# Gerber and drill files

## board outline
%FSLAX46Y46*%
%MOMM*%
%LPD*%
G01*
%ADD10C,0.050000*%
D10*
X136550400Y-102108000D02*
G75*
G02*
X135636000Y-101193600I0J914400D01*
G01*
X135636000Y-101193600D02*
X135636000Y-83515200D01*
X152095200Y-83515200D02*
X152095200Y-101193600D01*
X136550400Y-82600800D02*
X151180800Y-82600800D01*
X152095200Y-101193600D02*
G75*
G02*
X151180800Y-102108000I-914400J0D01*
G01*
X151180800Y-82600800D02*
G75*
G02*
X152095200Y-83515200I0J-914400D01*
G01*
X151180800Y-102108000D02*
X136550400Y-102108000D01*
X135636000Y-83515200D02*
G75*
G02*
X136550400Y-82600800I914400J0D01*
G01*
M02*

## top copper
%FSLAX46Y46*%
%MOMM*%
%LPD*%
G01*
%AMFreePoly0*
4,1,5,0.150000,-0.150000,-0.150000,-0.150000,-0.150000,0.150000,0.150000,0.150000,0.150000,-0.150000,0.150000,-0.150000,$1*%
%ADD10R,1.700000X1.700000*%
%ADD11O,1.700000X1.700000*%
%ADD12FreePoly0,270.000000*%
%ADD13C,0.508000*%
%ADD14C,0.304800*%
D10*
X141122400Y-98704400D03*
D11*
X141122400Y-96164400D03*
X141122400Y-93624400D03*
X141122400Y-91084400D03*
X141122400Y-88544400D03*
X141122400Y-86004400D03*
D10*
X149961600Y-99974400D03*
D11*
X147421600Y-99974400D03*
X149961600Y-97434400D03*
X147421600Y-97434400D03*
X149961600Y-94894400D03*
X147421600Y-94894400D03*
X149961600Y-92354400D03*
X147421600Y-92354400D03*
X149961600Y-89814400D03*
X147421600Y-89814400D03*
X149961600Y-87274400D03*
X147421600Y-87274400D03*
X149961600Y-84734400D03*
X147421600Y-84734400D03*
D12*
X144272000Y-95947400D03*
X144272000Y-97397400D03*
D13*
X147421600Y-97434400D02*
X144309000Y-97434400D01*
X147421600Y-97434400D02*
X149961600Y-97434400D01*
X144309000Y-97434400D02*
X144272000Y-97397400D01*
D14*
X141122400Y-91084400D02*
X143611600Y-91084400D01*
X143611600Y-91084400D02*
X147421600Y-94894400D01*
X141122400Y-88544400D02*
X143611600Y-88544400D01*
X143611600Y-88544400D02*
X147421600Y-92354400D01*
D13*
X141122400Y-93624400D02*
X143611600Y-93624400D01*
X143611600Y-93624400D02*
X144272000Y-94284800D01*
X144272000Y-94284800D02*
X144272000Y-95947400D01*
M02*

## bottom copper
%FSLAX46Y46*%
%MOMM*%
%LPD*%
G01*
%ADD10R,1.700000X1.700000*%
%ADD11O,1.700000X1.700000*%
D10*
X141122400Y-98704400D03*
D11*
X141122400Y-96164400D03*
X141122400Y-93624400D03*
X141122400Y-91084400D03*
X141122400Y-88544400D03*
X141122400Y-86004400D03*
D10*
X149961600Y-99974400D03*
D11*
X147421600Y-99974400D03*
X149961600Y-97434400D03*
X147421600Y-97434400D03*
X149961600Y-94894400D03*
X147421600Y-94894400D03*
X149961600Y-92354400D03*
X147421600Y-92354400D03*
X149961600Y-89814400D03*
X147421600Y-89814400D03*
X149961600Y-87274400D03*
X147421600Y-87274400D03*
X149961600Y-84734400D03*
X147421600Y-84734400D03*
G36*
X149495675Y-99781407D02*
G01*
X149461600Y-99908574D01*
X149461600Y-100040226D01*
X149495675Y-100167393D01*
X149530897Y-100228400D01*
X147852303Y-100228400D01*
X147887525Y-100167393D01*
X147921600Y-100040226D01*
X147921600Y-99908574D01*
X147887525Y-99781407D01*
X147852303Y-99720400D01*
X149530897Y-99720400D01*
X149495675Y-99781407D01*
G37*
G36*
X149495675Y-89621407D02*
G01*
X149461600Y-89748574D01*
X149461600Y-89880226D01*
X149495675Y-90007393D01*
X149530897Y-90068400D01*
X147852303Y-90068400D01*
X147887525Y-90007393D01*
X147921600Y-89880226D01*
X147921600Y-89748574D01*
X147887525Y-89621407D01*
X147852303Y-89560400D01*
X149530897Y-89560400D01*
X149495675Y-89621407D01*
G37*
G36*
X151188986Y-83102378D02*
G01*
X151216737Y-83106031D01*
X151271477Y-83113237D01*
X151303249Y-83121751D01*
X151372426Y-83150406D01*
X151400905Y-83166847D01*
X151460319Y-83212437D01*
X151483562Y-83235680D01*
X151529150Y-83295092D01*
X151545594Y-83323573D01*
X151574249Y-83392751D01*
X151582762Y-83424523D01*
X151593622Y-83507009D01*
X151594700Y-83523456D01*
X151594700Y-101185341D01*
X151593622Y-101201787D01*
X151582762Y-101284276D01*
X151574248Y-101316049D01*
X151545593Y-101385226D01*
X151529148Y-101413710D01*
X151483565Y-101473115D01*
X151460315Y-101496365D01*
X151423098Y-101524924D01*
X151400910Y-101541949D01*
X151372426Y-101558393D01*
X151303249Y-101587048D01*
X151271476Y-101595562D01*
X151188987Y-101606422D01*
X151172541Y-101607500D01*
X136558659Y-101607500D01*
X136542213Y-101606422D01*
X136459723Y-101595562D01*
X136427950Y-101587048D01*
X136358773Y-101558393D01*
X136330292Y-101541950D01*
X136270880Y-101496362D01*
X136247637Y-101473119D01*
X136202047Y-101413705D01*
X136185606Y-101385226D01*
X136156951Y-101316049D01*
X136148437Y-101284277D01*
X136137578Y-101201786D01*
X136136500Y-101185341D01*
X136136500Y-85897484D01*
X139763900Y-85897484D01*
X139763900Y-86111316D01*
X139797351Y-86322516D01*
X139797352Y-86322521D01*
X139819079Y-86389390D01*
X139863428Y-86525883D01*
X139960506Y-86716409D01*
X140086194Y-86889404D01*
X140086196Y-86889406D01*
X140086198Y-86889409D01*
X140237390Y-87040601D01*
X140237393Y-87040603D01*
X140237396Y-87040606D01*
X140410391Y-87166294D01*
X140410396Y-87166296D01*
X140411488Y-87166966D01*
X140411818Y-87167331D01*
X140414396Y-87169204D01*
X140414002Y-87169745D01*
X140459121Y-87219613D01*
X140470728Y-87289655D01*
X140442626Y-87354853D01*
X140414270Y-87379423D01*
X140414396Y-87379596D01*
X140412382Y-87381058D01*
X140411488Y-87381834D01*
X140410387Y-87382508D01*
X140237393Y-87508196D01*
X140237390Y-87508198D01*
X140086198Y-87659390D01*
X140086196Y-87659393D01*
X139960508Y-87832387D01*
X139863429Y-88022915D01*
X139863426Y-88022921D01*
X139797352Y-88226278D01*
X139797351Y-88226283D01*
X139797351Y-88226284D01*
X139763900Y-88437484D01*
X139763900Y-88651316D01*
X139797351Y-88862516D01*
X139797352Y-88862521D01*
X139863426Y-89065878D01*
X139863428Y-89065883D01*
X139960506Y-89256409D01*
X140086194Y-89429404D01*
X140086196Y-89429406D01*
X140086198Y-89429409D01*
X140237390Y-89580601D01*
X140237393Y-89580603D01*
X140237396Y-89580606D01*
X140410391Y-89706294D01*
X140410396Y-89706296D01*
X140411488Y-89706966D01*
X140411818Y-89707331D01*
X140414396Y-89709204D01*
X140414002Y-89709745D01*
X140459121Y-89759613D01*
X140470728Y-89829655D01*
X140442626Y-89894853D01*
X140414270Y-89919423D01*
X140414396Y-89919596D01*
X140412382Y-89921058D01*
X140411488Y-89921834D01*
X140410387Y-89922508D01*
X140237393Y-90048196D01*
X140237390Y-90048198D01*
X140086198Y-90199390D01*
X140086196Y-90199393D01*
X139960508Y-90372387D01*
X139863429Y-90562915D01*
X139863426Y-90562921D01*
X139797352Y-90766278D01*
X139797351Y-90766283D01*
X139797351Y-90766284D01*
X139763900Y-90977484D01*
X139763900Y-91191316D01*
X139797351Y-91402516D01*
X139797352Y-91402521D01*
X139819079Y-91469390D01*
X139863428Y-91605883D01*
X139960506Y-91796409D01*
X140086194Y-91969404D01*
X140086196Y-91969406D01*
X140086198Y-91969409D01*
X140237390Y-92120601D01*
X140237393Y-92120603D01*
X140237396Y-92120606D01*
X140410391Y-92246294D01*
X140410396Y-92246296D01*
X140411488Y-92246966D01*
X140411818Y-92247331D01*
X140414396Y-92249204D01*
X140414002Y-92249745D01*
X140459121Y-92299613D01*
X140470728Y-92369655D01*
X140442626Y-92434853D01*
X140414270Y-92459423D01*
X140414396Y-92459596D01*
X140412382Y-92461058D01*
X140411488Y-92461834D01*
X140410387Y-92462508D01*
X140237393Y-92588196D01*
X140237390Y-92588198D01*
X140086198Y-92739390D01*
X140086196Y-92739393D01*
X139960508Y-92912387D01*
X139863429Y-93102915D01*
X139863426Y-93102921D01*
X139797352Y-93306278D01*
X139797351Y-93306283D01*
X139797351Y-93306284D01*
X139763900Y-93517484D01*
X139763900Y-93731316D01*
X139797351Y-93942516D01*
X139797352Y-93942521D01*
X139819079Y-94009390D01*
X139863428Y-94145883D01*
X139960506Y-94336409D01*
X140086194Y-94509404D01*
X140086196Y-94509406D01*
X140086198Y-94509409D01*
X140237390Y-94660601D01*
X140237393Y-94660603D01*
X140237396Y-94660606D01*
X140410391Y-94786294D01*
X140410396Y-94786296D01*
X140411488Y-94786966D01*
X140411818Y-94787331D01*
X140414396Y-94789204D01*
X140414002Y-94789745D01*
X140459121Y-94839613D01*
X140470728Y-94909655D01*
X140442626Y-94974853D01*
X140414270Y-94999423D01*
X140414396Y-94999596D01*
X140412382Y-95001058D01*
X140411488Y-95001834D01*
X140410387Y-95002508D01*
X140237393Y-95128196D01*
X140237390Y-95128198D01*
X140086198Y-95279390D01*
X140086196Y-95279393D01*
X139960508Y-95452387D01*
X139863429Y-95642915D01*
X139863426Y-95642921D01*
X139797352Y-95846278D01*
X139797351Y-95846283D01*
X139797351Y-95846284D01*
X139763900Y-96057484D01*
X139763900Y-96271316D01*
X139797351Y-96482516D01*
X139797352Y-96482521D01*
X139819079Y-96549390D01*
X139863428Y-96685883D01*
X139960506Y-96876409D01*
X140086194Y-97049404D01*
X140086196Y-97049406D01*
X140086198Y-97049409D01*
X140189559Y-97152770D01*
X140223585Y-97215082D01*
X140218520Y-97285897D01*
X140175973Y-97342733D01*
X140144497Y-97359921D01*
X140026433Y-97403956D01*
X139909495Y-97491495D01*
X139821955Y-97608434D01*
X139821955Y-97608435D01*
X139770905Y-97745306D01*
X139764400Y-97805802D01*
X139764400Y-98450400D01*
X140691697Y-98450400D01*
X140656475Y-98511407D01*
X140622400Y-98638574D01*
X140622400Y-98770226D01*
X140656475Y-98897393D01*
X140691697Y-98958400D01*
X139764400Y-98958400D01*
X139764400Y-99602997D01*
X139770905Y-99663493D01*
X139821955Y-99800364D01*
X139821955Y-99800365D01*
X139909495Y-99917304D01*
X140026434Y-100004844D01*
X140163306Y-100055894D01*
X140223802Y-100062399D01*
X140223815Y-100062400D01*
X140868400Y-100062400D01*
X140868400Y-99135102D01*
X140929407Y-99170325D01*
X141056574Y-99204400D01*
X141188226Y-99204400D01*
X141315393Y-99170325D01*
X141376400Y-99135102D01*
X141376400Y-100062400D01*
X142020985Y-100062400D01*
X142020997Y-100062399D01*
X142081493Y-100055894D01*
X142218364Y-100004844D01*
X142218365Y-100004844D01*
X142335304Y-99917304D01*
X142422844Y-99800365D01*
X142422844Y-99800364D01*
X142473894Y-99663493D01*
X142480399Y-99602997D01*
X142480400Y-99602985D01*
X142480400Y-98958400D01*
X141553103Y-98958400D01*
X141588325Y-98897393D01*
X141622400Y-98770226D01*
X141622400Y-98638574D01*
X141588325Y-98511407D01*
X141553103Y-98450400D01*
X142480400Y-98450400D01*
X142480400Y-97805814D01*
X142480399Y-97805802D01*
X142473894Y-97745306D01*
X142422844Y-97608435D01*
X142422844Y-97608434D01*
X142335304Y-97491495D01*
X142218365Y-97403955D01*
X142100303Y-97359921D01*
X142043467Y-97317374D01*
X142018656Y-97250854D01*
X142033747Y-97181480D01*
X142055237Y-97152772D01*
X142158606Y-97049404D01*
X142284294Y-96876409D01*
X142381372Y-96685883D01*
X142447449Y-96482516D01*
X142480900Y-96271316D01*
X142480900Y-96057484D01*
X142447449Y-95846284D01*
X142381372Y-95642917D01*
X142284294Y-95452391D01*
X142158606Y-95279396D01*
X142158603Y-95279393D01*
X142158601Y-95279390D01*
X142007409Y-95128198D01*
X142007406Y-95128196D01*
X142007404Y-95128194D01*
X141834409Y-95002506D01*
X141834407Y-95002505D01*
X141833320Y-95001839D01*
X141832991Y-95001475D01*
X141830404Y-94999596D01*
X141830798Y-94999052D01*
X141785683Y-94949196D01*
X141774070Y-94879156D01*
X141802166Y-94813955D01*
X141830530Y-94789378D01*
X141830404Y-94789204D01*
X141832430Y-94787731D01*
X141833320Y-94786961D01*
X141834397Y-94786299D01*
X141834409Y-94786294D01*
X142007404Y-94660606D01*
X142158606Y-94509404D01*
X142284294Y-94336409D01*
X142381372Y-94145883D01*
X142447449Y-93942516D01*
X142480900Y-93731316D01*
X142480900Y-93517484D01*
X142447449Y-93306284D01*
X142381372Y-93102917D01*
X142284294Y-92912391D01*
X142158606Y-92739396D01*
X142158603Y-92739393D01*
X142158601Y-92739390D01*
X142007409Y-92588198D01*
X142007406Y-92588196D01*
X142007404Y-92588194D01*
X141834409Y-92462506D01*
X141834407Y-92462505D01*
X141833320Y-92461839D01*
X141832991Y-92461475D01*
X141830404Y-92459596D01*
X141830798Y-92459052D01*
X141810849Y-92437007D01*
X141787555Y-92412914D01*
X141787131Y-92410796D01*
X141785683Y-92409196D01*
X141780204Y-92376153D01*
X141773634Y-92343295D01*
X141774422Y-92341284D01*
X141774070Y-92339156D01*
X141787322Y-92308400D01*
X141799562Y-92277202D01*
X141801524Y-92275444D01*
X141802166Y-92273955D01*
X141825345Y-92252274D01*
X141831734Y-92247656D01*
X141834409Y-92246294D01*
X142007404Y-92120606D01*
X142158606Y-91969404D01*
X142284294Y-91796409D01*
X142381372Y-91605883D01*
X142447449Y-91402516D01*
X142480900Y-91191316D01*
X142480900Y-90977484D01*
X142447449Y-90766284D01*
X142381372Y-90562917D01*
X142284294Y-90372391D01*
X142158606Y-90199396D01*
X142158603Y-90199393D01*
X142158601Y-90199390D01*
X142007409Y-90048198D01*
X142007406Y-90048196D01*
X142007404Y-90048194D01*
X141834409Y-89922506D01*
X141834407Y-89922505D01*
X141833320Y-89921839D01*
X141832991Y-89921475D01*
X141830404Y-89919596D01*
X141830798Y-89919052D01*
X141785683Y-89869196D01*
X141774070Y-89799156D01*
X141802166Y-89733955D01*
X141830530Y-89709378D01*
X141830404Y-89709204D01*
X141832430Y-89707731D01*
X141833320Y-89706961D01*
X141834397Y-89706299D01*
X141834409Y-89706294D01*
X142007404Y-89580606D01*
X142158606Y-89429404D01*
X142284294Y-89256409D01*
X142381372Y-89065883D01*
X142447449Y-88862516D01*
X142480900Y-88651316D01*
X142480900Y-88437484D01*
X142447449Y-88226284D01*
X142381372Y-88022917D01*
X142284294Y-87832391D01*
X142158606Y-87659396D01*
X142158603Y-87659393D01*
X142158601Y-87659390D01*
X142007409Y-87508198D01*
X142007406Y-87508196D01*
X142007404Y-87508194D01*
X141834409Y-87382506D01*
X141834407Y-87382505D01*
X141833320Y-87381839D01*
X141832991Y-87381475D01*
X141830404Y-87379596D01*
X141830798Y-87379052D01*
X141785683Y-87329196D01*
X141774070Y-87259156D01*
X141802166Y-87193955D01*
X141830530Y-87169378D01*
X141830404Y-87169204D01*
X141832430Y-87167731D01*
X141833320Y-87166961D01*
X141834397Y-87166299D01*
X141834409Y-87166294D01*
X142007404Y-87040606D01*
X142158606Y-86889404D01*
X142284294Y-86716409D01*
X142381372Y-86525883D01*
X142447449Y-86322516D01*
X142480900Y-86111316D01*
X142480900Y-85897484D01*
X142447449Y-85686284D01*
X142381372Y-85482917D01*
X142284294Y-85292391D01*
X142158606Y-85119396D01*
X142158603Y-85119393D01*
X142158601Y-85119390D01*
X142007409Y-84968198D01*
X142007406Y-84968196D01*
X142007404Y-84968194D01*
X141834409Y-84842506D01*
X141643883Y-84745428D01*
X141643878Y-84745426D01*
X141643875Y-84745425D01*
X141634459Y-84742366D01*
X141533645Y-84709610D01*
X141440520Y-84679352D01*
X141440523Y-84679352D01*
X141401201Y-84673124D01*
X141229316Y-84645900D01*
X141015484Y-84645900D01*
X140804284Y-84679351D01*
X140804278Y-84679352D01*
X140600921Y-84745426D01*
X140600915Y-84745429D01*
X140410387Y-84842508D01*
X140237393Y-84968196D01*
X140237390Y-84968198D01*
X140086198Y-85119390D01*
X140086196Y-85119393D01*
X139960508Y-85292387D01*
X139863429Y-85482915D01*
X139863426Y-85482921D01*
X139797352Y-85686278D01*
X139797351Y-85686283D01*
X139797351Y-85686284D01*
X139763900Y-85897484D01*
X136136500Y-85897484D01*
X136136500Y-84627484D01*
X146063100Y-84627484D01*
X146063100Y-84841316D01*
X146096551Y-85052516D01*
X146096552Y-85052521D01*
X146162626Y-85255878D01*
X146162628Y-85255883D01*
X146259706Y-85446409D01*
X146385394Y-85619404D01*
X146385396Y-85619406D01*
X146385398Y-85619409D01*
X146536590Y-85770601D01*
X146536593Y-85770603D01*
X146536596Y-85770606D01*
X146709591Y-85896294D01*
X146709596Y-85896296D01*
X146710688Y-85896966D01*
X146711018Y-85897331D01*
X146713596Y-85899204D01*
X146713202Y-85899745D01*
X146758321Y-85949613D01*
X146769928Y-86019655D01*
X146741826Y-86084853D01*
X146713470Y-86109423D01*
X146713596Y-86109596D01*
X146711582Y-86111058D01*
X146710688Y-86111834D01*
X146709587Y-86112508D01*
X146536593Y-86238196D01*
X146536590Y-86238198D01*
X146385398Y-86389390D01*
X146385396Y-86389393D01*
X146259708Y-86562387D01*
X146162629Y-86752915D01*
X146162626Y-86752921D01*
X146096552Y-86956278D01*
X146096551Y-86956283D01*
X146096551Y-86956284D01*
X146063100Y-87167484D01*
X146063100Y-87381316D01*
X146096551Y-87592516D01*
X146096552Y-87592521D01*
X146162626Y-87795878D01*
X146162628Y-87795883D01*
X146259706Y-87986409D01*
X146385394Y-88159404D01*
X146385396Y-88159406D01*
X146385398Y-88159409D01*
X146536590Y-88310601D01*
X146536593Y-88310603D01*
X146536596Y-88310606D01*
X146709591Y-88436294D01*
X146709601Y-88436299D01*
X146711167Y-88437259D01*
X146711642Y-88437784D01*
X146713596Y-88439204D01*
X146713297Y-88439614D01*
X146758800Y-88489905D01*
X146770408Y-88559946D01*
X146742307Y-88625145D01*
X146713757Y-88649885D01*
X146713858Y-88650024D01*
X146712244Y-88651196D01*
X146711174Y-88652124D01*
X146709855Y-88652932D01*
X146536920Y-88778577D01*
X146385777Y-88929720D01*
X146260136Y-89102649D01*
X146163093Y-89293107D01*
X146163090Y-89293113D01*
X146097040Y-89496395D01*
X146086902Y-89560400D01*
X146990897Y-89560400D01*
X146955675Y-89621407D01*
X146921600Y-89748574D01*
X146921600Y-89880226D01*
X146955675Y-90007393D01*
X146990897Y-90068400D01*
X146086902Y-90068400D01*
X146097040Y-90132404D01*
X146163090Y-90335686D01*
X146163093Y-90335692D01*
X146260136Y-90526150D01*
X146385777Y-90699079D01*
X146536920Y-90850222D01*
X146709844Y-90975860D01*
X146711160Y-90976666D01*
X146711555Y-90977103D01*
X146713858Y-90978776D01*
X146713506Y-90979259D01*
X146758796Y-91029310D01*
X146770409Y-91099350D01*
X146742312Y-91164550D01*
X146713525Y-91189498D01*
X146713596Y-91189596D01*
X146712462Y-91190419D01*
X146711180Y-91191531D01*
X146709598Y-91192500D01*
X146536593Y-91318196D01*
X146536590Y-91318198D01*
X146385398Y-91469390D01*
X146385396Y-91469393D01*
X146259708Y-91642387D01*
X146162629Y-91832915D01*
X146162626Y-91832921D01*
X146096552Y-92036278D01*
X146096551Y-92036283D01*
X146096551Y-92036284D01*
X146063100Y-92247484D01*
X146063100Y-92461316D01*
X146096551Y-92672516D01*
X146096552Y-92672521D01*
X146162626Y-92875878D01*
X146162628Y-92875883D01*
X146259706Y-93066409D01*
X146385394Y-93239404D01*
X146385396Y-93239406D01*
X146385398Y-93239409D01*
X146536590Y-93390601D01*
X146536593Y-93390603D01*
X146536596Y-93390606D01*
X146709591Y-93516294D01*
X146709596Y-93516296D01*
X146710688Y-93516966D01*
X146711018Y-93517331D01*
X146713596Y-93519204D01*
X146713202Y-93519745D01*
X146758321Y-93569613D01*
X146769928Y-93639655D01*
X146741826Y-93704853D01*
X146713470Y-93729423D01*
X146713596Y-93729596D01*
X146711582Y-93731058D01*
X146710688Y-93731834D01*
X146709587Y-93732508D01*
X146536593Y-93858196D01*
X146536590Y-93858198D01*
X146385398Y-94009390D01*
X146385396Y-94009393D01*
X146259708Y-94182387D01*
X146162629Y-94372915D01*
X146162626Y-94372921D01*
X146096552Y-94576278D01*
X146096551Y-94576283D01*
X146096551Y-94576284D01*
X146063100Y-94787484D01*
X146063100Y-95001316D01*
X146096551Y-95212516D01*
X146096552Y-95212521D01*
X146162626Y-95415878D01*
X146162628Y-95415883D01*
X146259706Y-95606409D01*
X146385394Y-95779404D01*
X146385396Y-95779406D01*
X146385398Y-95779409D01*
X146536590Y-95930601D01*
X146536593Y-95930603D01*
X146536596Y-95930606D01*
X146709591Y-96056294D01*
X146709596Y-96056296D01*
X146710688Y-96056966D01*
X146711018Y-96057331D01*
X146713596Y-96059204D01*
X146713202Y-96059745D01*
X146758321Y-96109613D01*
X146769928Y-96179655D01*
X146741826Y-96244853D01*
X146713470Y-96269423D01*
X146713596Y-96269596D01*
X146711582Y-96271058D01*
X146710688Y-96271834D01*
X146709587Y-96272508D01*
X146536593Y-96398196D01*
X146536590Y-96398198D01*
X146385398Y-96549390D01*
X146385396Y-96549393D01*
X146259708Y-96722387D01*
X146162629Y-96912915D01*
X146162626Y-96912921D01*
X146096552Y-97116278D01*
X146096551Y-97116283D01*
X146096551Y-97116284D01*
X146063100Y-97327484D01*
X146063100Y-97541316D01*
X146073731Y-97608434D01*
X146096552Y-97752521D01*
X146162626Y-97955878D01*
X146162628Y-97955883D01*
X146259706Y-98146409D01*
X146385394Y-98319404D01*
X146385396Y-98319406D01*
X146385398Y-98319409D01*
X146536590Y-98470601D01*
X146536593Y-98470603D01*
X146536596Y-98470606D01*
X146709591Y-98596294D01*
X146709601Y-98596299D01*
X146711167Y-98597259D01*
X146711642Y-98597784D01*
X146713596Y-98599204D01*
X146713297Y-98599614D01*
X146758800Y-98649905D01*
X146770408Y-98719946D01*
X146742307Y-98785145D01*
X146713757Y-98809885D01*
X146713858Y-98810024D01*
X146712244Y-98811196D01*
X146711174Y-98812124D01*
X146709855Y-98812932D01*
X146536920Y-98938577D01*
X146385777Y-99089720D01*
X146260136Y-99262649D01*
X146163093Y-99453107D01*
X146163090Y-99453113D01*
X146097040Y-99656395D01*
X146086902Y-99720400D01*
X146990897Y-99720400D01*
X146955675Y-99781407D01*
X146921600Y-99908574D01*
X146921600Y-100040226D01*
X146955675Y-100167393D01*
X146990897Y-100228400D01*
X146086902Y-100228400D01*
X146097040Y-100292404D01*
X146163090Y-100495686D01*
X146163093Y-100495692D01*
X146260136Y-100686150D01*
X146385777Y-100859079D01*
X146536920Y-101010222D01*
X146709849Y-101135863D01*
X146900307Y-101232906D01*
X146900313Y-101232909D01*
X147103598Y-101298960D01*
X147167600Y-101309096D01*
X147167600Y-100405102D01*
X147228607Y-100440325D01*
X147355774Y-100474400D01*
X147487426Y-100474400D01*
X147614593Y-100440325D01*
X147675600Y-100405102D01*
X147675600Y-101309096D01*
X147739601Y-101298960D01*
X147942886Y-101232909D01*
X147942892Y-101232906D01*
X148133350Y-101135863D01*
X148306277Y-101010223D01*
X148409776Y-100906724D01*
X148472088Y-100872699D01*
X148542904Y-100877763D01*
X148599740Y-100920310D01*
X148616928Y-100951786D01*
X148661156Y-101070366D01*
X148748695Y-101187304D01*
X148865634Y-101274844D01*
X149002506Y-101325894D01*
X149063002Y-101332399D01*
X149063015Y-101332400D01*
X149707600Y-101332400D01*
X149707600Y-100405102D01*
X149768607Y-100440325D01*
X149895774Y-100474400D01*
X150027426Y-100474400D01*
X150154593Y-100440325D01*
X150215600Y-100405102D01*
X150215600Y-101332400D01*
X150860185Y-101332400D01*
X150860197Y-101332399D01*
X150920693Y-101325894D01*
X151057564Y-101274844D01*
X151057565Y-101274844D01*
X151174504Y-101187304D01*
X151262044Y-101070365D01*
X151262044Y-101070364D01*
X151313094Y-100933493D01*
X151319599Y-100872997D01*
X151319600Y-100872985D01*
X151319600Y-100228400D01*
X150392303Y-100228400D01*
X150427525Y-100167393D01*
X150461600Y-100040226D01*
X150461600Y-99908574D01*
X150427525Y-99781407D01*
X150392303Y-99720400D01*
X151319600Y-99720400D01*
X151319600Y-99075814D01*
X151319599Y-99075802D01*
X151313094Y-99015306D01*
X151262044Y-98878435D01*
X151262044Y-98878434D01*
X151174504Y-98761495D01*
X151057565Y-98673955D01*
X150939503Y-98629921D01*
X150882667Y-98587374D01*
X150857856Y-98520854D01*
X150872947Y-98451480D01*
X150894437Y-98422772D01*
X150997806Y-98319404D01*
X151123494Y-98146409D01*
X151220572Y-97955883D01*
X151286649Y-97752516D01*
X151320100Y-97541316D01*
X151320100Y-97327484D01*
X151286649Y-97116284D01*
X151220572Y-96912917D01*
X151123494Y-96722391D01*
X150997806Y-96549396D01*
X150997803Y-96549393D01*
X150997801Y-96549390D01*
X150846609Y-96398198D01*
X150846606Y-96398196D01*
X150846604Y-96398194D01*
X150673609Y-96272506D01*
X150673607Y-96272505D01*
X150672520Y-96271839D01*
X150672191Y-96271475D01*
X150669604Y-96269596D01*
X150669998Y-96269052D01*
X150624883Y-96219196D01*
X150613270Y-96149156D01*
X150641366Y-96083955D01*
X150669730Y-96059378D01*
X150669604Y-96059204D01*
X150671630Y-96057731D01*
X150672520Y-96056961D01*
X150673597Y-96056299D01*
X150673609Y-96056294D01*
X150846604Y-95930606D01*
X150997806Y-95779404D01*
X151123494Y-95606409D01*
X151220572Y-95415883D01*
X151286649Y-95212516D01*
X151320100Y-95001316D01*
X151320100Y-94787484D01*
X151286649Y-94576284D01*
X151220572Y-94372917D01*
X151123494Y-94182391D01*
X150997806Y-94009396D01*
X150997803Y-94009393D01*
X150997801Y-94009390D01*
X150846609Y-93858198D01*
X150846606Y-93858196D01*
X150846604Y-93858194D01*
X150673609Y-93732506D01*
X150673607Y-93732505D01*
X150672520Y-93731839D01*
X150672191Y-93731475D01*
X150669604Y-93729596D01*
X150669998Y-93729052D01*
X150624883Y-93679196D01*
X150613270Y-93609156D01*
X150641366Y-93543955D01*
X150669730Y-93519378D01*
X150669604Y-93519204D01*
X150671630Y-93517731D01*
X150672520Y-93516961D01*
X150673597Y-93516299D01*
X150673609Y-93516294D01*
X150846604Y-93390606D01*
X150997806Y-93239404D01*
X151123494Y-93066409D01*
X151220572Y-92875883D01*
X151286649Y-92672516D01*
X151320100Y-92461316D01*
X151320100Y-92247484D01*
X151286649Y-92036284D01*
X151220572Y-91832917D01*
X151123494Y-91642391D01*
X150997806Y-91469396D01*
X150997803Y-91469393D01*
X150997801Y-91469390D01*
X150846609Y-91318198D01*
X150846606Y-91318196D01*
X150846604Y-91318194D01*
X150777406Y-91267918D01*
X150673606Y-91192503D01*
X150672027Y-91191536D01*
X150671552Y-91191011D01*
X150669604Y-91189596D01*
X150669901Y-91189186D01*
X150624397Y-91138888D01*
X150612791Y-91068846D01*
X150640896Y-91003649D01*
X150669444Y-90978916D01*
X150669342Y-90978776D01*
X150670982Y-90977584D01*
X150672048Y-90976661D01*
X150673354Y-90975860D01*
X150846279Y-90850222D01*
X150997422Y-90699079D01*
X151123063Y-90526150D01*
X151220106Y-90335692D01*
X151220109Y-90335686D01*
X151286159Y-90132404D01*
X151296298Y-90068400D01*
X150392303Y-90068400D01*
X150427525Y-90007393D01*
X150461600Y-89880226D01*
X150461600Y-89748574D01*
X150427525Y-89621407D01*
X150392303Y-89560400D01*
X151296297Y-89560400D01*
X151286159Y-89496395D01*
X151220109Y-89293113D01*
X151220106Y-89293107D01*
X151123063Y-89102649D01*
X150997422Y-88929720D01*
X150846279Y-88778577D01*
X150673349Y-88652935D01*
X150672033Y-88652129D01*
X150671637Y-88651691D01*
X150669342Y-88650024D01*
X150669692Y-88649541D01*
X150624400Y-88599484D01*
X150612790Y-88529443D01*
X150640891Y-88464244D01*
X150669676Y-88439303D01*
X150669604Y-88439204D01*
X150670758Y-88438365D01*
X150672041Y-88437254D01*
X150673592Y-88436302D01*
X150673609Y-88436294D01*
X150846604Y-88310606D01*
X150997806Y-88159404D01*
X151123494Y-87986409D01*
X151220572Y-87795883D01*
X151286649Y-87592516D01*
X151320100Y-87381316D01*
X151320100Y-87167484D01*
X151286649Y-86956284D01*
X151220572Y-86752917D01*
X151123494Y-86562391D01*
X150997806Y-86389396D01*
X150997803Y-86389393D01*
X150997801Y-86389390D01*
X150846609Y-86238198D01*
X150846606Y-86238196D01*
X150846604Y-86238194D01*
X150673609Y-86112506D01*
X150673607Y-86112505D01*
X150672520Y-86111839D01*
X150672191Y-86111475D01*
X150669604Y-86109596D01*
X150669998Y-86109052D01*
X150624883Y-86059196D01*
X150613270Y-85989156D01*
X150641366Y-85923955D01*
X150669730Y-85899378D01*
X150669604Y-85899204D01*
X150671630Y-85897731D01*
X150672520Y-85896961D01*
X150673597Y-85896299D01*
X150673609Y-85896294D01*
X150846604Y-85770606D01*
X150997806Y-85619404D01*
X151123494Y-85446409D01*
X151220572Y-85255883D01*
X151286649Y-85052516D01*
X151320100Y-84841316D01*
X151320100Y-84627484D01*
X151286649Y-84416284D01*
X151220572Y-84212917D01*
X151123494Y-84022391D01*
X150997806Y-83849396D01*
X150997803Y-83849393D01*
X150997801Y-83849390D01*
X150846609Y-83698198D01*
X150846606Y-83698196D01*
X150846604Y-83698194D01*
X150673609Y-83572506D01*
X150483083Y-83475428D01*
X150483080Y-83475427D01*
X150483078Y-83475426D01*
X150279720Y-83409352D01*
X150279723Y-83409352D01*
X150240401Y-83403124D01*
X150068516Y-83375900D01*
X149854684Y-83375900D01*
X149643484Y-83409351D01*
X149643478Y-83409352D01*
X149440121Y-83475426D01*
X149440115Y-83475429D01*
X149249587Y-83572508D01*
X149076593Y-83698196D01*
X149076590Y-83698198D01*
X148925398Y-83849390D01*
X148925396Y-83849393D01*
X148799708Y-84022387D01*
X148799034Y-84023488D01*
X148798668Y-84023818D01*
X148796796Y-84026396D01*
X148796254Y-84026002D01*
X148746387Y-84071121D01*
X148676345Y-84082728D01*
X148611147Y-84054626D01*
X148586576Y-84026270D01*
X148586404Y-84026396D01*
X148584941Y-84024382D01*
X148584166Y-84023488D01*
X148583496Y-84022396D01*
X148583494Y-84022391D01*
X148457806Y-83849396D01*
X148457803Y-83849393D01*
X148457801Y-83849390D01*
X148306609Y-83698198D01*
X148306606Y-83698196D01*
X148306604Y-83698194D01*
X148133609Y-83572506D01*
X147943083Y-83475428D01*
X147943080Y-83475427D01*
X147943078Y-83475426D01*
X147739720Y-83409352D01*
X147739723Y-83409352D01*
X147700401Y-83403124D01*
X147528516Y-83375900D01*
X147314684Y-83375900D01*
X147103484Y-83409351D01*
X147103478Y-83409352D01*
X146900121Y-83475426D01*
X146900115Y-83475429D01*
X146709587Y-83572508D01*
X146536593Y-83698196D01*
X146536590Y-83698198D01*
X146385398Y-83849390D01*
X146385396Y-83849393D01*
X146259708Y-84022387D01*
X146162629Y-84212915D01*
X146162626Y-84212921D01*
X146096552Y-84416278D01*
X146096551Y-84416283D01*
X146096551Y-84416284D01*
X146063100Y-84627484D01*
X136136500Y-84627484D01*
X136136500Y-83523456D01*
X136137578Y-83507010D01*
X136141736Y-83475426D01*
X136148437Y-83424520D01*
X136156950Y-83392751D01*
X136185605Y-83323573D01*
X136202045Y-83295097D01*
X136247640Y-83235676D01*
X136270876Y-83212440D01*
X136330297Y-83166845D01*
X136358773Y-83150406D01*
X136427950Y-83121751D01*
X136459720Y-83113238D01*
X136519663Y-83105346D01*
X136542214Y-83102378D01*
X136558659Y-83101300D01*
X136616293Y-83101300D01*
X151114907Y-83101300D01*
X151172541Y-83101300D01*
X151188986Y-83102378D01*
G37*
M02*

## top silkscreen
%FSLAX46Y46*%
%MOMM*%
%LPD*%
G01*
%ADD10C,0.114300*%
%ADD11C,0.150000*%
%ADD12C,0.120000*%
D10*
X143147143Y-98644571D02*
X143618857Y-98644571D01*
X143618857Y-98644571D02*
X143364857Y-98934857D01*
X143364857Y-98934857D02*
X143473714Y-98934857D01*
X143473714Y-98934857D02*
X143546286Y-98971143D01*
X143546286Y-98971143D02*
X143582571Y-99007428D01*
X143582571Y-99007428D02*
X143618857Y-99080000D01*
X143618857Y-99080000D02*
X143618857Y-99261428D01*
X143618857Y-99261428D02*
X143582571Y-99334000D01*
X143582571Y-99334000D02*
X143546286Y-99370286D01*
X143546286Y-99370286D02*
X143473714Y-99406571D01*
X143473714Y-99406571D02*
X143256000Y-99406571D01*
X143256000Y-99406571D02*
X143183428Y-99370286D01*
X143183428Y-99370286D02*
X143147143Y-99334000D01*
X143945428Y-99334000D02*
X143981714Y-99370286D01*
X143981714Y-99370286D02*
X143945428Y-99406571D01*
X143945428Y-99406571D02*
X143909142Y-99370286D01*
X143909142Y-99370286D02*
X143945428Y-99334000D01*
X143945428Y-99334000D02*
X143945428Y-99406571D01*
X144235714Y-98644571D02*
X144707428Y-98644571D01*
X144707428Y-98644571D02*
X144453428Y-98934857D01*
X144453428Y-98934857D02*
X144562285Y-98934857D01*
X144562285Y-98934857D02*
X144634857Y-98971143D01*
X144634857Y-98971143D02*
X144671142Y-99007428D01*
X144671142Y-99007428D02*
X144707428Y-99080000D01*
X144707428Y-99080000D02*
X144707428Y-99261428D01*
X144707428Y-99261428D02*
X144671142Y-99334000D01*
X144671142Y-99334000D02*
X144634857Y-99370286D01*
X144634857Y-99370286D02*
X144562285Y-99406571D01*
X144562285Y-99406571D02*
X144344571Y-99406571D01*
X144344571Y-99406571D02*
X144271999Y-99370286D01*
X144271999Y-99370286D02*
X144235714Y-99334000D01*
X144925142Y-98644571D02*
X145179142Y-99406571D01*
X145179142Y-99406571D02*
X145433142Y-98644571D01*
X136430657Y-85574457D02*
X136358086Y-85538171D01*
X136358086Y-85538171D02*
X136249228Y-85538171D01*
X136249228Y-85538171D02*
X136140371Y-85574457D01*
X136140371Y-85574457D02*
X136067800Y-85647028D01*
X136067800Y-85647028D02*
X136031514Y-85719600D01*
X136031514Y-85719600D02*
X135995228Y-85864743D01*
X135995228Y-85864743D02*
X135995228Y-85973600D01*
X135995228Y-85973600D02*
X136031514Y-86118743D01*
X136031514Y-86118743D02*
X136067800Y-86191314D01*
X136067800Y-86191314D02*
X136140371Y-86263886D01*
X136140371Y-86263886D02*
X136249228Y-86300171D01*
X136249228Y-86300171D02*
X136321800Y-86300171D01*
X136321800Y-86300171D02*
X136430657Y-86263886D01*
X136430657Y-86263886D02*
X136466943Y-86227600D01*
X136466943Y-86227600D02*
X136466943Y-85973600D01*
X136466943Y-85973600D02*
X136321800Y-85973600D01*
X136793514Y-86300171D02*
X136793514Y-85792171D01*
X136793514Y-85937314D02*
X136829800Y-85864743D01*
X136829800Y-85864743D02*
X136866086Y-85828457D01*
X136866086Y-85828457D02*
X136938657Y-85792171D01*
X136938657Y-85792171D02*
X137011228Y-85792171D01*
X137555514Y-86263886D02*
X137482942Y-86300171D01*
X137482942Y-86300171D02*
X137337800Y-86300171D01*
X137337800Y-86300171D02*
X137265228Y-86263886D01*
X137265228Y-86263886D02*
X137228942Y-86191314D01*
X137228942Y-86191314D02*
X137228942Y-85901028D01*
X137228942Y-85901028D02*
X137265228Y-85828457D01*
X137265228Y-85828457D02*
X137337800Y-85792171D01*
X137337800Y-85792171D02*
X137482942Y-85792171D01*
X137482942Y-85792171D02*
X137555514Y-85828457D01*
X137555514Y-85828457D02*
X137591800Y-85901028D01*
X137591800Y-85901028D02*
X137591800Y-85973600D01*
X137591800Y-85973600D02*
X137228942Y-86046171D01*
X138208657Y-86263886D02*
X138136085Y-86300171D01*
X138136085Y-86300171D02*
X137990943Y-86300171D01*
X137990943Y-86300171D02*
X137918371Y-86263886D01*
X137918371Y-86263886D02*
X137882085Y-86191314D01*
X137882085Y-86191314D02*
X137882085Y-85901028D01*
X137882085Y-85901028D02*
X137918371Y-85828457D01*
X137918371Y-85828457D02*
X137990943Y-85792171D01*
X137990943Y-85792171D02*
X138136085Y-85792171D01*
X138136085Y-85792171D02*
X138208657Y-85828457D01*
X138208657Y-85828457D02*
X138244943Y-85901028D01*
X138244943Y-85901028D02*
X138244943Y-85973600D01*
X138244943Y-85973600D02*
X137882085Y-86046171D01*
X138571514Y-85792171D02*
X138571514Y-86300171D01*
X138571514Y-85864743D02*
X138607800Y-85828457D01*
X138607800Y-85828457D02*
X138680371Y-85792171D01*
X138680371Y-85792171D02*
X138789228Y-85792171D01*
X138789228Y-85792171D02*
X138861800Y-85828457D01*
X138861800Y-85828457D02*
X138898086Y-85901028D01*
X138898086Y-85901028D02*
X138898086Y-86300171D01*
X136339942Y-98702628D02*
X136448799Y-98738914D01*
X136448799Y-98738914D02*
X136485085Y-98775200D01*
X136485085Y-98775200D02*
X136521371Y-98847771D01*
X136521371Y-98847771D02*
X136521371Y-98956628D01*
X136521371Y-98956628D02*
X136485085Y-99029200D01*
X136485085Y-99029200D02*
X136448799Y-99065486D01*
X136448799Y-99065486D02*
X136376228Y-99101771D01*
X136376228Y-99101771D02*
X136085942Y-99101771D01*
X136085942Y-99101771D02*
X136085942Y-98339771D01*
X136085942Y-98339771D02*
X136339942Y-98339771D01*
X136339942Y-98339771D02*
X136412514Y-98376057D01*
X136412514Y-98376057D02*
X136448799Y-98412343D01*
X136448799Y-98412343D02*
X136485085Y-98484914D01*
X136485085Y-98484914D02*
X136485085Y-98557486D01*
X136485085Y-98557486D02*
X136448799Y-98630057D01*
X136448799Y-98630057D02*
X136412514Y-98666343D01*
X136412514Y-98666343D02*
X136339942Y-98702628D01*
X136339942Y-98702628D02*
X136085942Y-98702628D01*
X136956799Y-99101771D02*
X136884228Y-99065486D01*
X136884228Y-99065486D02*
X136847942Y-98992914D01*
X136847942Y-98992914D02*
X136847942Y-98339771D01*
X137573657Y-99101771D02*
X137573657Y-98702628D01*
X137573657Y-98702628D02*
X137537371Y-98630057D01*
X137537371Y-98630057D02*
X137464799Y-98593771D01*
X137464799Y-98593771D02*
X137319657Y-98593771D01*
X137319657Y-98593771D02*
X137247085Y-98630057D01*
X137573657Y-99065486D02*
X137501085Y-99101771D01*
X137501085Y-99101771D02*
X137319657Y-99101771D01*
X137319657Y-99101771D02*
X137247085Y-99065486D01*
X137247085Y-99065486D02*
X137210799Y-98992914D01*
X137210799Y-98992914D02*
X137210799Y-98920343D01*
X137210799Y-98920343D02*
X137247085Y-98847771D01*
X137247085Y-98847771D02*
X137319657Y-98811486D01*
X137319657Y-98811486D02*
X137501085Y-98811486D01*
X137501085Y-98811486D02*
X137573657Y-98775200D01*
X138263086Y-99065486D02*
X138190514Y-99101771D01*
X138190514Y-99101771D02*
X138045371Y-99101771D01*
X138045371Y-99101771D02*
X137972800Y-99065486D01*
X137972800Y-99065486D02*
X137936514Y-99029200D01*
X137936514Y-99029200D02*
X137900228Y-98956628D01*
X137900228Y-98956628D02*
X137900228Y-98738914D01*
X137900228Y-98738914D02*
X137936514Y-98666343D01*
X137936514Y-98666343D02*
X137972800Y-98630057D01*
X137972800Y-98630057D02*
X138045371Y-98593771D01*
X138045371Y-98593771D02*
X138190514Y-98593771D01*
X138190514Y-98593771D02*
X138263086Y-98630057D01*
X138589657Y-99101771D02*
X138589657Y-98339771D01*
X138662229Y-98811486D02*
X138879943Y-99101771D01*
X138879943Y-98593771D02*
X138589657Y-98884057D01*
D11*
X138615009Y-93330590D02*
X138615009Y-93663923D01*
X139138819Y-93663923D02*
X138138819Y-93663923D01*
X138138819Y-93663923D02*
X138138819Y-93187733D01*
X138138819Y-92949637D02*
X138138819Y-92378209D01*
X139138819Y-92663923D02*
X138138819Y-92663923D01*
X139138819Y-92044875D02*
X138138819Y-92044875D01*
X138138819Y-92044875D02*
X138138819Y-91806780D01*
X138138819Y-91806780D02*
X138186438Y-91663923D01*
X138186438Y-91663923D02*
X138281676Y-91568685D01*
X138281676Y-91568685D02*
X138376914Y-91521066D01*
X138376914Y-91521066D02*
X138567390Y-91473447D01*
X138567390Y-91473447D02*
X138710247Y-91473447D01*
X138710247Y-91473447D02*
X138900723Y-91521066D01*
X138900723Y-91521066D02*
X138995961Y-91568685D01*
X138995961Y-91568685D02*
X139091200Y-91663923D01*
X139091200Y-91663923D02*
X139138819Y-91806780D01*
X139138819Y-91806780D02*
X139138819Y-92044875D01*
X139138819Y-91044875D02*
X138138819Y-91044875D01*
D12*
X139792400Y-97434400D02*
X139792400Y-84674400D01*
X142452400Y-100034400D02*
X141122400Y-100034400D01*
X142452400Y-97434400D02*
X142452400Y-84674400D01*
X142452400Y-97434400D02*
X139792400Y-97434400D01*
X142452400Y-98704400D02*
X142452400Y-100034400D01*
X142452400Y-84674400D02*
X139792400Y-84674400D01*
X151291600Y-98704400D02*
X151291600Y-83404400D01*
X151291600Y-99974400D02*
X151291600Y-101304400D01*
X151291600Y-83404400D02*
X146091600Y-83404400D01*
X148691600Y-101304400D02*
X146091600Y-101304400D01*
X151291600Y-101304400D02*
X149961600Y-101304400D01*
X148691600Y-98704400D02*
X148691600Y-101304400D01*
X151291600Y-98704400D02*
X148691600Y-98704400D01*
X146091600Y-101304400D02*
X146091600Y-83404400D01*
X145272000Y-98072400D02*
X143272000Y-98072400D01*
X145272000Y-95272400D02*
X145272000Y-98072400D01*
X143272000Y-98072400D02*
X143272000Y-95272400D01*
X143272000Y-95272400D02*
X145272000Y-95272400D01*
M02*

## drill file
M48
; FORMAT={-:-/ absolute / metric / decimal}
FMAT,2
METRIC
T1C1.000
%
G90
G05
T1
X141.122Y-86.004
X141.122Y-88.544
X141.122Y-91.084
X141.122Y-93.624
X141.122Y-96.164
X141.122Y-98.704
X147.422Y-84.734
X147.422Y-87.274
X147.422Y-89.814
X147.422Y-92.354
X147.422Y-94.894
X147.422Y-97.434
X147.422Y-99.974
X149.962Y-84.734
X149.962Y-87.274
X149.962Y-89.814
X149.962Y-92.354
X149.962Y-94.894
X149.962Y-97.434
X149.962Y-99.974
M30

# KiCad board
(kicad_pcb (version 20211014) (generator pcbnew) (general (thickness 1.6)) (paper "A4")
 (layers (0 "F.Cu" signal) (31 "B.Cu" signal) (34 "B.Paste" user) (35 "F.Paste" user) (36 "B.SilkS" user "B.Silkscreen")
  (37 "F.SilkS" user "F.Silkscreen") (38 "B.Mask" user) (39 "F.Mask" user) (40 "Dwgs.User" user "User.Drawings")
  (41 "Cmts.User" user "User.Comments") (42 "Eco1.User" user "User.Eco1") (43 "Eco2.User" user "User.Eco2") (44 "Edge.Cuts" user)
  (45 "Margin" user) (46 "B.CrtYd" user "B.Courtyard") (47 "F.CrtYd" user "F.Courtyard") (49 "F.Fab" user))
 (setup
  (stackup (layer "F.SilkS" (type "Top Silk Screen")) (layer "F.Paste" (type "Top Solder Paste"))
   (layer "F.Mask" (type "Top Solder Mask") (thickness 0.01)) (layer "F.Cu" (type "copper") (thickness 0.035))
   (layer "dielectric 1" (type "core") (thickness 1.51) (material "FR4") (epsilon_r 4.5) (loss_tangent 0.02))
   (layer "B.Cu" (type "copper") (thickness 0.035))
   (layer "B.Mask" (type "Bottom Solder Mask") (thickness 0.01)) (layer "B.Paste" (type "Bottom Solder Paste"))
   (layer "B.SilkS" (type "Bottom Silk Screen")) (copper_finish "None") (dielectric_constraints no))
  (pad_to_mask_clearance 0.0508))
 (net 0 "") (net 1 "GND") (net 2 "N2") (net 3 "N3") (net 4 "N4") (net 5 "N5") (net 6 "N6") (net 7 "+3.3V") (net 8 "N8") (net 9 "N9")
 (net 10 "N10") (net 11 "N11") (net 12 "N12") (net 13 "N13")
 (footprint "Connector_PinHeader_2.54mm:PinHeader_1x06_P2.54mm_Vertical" (layer "F.Cu") (at 141.1224 98.7044 180)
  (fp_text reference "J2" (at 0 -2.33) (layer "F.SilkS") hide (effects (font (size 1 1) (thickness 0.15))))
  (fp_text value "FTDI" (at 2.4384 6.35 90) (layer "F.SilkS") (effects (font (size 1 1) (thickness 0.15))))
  (fp_line (start 1.33 1.27) (end 1.33 14.03) (layer "F.SilkS") (width 0.12))
  (fp_line (start -1.33 -1.33) (end 0 -1.33) (layer "F.SilkS") (width 0.12))
  (fp_line (start -1.33 1.27) (end -1.33 14.03) (layer "F.SilkS") (width 0.12))
  (fp_line (start -1.33 1.27) (end 1.33 1.27) (layer "F.SilkS") (width 0.12))
  (fp_line (start -1.33 0) (end -1.33 -1.33) (layer "F.SilkS") (width 0.12))
  (fp_line (start -1.33 14.03) (end 1.33 14.03) (layer "F.SilkS") (width 0.12))
  (pad "1" thru_hole rect (at 0 0 180) (size 1.7 1.7) (drill 1) (layers *.Cu *.Mask) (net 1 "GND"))
  (pad "2" thru_hole oval (at 0 2.54 180) (size 1.7 1.7) (drill 1) (layers *.Cu *.Mask) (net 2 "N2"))
  (pad "3" thru_hole oval (at 0 5.08 180) (size 1.7 1.7) (drill 1) (layers *.Cu *.Mask) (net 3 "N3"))
  (pad "4" thru_hole oval (at 0 7.62 180) (size 1.7 1.7) (drill 1) (layers *.Cu *.Mask) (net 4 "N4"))
  (pad "5" thru_hole oval (at 0 10.16 180) (size 1.7 1.7) (drill 1) (layers *.Cu *.Mask) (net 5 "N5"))
  (pad "6" thru_hole oval (at 0 12.7 180) (size 1.7 1.7) (drill 1) (layers *.Cu *.Mask) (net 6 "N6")))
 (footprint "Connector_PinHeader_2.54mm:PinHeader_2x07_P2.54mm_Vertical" (layer "F.Cu") (at 149.9616 99.9744 180)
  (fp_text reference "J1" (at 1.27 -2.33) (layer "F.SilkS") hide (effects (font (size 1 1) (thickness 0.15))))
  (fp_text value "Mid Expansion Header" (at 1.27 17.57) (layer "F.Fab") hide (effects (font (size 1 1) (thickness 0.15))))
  (fp_line (start -1.33 1.27) (end -1.33 16.57) (layer "F.SilkS") (width 0.12))
  (fp_line (start -1.33 0) (end -1.33 -1.33) (layer "F.SilkS") (width 0.12))
  (fp_line (start -1.33 16.57) (end 3.87 16.57) (layer "F.SilkS") (width 0.12))
  (fp_line (start 1.27 -1.33) (end 3.87 -1.33) (layer "F.SilkS") (width 0.12))
  (fp_line (start -1.33 -1.33) (end 0 -1.33) (layer "F.SilkS") (width 0.12))
  (fp_line (start 1.27 1.27) (end 1.27 -1.33) (layer "F.SilkS") (width 0.12))
  (fp_line (start -1.33 1.27) (end 1.27 1.27) (layer "F.SilkS") (width 0.12))
  (fp_line (start 3.87 -1.33) (end 3.87 16.57) (layer "F.SilkS") (width 0.12))
  (pad "1" thru_hole rect (at 0 0 180) (size 1.7 1.7) (drill 1) (layers *.Cu *.Mask) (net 1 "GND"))
  (pad "2" thru_hole oval (at 2.54 0 180) (size 1.7 1.7) (drill 1) (layers *.Cu *.Mask) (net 1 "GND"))
  (pad "3" thru_hole oval (at 0 2.54 180) (size 1.7 1.7) (drill 1) (layers *.Cu *.Mask) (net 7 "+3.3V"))
  (pad "4" thru_hole oval (at 2.54 2.54 180) (size 1.7 1.7) (drill 1) (layers *.Cu *.Mask) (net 7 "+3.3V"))
  (pad "5" thru_hole oval (at 0 5.08 180) (size 1.7 1.7) (drill 1) (layers *.Cu *.Mask) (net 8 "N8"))
  (pad "6" thru_hole oval (at 2.54 5.08 180) (size 1.7 1.7) (drill 1) (layers *.Cu *.Mask) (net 4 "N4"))
  (pad "7" thru_hole oval (at 0 7.62 180) (size 1.7 1.7) (drill 1) (layers *.Cu *.Mask) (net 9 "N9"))
  (pad "8" thru_hole oval (at 2.54 7.62 180) (size 1.7 1.7) (drill 1) (layers *.Cu *.Mask) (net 5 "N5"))
  (pad "9" thru_hole oval (at 0 10.16 180) (size 1.7 1.7) (drill 1) (layers *.Cu *.Mask) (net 1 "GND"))
  (pad "10" thru_hole oval (at 2.54 10.16 180) (size 1.7 1.7) (drill 1) (layers *.Cu *.Mask) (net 1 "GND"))
  (pad "11" thru_hole oval (at 0 12.7 180) (size 1.7 1.7) (drill 1) (layers *.Cu *.Mask) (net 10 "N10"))
  (pad "12" thru_hole oval (at 2.54 12.7 180) (size 1.7 1.7) (drill 1) (layers *.Cu *.Mask) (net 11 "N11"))
  (pad "13" thru_hole oval (at 0 15.24 180) (size 1.7 1.7) (drill 1) (layers *.Cu *.Mask) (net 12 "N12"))
  (pad "14" thru_hole oval (at 2.54 15.24 180) (size 1.7 1.7) (drill 1) (layers *.Cu *.Mask) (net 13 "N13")))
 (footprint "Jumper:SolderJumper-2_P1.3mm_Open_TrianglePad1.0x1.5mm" (layer "F.Cu") (at 144.272 96.6724 -90)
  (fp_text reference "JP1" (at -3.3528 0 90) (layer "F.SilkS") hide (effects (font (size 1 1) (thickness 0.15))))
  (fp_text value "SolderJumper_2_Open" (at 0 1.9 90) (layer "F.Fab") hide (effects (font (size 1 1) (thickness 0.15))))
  (fp_line (start 1.4 -1) (end 1.4 1) (layer "F.SilkS") (width 0.12))
  (fp_line (start -1.4 -1) (end 1.4 -1) (layer "F.SilkS") (width 0.12))
  (fp_line (start 1.4 1) (end -1.4 1) (layer "F.SilkS") (width 0.12))
  (fp_line (start -1.4 1) (end -1.4 -1) (layer "F.SilkS") (width 0.12))
  (pad "1" smd custom (at -0.725 0 270) (size 0.3 0.3) (layers "F.Cu" "F.Mask") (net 3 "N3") (zone_connect 2)
   (options (clearance outline) (anchor rect)) (primitives))
  (pad "2" smd custom (at 0.725 0 270) (size 0.3 0.3) (layers "F.Cu" "F.Mask") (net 7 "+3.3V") (zone_connect 2)
   (options (clearance outline) (anchor rect)) (primitives)))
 (gr_arc (start 136.5504 102.108) (mid 135.903822 101.840178) (end 135.636 101.1936) (layer "Edge.Cuts") (width 0.05))
 (gr_line (start 135.636 101.1936) (end 135.636 83.5152) (layer "Edge.Cuts") (width 0.05))
 (gr_line (start 152.0952 83.5152) (end 152.0952 101.1936) (layer "Edge.Cuts") (width 0.05))
 (gr_line (start 136.5504 82.6008) (end 151.1808 82.6008) (layer "Edge.Cuts") (width 0.05))
 (gr_arc (start 152.0952 101.1936) (mid 151.827378 101.840178) (end 151.1808 102.108) (layer "Edge.Cuts") (width 0.05))
 (gr_arc (start 151.1808 82.6008) (mid 151.827378 82.868622) (end 152.0952 83.5152) (layer "Edge.Cuts") (width 0.05))
 (gr_line (start 151.1808 102.108) (end 136.5504 102.108) (layer "Edge.Cuts") (width 0.05))
 (gr_arc (start 135.636 83.5152) (mid 135.903822 82.868622) (end 136.5504 82.6008) (layer "Edge.Cuts") (width 0.05))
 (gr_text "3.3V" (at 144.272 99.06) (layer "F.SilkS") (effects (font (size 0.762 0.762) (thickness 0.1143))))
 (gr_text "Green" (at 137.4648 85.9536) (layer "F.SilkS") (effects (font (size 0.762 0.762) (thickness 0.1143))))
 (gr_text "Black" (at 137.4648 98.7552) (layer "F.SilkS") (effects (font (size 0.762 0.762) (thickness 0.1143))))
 (segment (start 147.4216 97.4344) (end 144.309 97.4344) (width 0.508) (layer "F.Cu") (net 7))
 (segment (start 147.4216 97.4344) (end 149.9616 97.4344) (width 0.508) (layer "F.Cu") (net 7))
 (segment (start 144.309 97.4344) (end 144.272 97.3974) (width 0.508) (layer "F.Cu") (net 7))
 (segment (start 141.1224 91.0844) (end 143.6116 91.0844) (width 0.3048) (layer "F.Cu") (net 4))
 (segment (start 143.6116 91.0844) (end 147.4216 94.8944) (width 0.3048) (layer "F.Cu") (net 4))
 (segment (start 141.1224 88.5444) (end 143.6116 88.5444) (width 0.3048) (layer "F.Cu") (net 5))
 (segment (start 143.6116 88.5444) (end 147.4216 92.3544) (width 0.3048) (layer "F.Cu") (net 5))
 (segment (start 141.1224 93.6244) (end 143.6116 93.6244) (width 0.508) (layer "F.Cu") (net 3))
 (segment (start 143.6116 93.6244) (end 144.272 94.2848) (width 0.508) (layer "F.Cu") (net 3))
 (segment (start 144.272 94.2848) (end 144.272 95.9474) (width 0.508) (layer "F.Cu") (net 3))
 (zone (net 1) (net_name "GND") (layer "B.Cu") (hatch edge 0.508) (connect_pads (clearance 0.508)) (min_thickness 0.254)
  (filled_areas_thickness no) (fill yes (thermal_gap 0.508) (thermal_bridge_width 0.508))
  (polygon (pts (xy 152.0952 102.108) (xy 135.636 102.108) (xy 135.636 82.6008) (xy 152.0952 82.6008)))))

